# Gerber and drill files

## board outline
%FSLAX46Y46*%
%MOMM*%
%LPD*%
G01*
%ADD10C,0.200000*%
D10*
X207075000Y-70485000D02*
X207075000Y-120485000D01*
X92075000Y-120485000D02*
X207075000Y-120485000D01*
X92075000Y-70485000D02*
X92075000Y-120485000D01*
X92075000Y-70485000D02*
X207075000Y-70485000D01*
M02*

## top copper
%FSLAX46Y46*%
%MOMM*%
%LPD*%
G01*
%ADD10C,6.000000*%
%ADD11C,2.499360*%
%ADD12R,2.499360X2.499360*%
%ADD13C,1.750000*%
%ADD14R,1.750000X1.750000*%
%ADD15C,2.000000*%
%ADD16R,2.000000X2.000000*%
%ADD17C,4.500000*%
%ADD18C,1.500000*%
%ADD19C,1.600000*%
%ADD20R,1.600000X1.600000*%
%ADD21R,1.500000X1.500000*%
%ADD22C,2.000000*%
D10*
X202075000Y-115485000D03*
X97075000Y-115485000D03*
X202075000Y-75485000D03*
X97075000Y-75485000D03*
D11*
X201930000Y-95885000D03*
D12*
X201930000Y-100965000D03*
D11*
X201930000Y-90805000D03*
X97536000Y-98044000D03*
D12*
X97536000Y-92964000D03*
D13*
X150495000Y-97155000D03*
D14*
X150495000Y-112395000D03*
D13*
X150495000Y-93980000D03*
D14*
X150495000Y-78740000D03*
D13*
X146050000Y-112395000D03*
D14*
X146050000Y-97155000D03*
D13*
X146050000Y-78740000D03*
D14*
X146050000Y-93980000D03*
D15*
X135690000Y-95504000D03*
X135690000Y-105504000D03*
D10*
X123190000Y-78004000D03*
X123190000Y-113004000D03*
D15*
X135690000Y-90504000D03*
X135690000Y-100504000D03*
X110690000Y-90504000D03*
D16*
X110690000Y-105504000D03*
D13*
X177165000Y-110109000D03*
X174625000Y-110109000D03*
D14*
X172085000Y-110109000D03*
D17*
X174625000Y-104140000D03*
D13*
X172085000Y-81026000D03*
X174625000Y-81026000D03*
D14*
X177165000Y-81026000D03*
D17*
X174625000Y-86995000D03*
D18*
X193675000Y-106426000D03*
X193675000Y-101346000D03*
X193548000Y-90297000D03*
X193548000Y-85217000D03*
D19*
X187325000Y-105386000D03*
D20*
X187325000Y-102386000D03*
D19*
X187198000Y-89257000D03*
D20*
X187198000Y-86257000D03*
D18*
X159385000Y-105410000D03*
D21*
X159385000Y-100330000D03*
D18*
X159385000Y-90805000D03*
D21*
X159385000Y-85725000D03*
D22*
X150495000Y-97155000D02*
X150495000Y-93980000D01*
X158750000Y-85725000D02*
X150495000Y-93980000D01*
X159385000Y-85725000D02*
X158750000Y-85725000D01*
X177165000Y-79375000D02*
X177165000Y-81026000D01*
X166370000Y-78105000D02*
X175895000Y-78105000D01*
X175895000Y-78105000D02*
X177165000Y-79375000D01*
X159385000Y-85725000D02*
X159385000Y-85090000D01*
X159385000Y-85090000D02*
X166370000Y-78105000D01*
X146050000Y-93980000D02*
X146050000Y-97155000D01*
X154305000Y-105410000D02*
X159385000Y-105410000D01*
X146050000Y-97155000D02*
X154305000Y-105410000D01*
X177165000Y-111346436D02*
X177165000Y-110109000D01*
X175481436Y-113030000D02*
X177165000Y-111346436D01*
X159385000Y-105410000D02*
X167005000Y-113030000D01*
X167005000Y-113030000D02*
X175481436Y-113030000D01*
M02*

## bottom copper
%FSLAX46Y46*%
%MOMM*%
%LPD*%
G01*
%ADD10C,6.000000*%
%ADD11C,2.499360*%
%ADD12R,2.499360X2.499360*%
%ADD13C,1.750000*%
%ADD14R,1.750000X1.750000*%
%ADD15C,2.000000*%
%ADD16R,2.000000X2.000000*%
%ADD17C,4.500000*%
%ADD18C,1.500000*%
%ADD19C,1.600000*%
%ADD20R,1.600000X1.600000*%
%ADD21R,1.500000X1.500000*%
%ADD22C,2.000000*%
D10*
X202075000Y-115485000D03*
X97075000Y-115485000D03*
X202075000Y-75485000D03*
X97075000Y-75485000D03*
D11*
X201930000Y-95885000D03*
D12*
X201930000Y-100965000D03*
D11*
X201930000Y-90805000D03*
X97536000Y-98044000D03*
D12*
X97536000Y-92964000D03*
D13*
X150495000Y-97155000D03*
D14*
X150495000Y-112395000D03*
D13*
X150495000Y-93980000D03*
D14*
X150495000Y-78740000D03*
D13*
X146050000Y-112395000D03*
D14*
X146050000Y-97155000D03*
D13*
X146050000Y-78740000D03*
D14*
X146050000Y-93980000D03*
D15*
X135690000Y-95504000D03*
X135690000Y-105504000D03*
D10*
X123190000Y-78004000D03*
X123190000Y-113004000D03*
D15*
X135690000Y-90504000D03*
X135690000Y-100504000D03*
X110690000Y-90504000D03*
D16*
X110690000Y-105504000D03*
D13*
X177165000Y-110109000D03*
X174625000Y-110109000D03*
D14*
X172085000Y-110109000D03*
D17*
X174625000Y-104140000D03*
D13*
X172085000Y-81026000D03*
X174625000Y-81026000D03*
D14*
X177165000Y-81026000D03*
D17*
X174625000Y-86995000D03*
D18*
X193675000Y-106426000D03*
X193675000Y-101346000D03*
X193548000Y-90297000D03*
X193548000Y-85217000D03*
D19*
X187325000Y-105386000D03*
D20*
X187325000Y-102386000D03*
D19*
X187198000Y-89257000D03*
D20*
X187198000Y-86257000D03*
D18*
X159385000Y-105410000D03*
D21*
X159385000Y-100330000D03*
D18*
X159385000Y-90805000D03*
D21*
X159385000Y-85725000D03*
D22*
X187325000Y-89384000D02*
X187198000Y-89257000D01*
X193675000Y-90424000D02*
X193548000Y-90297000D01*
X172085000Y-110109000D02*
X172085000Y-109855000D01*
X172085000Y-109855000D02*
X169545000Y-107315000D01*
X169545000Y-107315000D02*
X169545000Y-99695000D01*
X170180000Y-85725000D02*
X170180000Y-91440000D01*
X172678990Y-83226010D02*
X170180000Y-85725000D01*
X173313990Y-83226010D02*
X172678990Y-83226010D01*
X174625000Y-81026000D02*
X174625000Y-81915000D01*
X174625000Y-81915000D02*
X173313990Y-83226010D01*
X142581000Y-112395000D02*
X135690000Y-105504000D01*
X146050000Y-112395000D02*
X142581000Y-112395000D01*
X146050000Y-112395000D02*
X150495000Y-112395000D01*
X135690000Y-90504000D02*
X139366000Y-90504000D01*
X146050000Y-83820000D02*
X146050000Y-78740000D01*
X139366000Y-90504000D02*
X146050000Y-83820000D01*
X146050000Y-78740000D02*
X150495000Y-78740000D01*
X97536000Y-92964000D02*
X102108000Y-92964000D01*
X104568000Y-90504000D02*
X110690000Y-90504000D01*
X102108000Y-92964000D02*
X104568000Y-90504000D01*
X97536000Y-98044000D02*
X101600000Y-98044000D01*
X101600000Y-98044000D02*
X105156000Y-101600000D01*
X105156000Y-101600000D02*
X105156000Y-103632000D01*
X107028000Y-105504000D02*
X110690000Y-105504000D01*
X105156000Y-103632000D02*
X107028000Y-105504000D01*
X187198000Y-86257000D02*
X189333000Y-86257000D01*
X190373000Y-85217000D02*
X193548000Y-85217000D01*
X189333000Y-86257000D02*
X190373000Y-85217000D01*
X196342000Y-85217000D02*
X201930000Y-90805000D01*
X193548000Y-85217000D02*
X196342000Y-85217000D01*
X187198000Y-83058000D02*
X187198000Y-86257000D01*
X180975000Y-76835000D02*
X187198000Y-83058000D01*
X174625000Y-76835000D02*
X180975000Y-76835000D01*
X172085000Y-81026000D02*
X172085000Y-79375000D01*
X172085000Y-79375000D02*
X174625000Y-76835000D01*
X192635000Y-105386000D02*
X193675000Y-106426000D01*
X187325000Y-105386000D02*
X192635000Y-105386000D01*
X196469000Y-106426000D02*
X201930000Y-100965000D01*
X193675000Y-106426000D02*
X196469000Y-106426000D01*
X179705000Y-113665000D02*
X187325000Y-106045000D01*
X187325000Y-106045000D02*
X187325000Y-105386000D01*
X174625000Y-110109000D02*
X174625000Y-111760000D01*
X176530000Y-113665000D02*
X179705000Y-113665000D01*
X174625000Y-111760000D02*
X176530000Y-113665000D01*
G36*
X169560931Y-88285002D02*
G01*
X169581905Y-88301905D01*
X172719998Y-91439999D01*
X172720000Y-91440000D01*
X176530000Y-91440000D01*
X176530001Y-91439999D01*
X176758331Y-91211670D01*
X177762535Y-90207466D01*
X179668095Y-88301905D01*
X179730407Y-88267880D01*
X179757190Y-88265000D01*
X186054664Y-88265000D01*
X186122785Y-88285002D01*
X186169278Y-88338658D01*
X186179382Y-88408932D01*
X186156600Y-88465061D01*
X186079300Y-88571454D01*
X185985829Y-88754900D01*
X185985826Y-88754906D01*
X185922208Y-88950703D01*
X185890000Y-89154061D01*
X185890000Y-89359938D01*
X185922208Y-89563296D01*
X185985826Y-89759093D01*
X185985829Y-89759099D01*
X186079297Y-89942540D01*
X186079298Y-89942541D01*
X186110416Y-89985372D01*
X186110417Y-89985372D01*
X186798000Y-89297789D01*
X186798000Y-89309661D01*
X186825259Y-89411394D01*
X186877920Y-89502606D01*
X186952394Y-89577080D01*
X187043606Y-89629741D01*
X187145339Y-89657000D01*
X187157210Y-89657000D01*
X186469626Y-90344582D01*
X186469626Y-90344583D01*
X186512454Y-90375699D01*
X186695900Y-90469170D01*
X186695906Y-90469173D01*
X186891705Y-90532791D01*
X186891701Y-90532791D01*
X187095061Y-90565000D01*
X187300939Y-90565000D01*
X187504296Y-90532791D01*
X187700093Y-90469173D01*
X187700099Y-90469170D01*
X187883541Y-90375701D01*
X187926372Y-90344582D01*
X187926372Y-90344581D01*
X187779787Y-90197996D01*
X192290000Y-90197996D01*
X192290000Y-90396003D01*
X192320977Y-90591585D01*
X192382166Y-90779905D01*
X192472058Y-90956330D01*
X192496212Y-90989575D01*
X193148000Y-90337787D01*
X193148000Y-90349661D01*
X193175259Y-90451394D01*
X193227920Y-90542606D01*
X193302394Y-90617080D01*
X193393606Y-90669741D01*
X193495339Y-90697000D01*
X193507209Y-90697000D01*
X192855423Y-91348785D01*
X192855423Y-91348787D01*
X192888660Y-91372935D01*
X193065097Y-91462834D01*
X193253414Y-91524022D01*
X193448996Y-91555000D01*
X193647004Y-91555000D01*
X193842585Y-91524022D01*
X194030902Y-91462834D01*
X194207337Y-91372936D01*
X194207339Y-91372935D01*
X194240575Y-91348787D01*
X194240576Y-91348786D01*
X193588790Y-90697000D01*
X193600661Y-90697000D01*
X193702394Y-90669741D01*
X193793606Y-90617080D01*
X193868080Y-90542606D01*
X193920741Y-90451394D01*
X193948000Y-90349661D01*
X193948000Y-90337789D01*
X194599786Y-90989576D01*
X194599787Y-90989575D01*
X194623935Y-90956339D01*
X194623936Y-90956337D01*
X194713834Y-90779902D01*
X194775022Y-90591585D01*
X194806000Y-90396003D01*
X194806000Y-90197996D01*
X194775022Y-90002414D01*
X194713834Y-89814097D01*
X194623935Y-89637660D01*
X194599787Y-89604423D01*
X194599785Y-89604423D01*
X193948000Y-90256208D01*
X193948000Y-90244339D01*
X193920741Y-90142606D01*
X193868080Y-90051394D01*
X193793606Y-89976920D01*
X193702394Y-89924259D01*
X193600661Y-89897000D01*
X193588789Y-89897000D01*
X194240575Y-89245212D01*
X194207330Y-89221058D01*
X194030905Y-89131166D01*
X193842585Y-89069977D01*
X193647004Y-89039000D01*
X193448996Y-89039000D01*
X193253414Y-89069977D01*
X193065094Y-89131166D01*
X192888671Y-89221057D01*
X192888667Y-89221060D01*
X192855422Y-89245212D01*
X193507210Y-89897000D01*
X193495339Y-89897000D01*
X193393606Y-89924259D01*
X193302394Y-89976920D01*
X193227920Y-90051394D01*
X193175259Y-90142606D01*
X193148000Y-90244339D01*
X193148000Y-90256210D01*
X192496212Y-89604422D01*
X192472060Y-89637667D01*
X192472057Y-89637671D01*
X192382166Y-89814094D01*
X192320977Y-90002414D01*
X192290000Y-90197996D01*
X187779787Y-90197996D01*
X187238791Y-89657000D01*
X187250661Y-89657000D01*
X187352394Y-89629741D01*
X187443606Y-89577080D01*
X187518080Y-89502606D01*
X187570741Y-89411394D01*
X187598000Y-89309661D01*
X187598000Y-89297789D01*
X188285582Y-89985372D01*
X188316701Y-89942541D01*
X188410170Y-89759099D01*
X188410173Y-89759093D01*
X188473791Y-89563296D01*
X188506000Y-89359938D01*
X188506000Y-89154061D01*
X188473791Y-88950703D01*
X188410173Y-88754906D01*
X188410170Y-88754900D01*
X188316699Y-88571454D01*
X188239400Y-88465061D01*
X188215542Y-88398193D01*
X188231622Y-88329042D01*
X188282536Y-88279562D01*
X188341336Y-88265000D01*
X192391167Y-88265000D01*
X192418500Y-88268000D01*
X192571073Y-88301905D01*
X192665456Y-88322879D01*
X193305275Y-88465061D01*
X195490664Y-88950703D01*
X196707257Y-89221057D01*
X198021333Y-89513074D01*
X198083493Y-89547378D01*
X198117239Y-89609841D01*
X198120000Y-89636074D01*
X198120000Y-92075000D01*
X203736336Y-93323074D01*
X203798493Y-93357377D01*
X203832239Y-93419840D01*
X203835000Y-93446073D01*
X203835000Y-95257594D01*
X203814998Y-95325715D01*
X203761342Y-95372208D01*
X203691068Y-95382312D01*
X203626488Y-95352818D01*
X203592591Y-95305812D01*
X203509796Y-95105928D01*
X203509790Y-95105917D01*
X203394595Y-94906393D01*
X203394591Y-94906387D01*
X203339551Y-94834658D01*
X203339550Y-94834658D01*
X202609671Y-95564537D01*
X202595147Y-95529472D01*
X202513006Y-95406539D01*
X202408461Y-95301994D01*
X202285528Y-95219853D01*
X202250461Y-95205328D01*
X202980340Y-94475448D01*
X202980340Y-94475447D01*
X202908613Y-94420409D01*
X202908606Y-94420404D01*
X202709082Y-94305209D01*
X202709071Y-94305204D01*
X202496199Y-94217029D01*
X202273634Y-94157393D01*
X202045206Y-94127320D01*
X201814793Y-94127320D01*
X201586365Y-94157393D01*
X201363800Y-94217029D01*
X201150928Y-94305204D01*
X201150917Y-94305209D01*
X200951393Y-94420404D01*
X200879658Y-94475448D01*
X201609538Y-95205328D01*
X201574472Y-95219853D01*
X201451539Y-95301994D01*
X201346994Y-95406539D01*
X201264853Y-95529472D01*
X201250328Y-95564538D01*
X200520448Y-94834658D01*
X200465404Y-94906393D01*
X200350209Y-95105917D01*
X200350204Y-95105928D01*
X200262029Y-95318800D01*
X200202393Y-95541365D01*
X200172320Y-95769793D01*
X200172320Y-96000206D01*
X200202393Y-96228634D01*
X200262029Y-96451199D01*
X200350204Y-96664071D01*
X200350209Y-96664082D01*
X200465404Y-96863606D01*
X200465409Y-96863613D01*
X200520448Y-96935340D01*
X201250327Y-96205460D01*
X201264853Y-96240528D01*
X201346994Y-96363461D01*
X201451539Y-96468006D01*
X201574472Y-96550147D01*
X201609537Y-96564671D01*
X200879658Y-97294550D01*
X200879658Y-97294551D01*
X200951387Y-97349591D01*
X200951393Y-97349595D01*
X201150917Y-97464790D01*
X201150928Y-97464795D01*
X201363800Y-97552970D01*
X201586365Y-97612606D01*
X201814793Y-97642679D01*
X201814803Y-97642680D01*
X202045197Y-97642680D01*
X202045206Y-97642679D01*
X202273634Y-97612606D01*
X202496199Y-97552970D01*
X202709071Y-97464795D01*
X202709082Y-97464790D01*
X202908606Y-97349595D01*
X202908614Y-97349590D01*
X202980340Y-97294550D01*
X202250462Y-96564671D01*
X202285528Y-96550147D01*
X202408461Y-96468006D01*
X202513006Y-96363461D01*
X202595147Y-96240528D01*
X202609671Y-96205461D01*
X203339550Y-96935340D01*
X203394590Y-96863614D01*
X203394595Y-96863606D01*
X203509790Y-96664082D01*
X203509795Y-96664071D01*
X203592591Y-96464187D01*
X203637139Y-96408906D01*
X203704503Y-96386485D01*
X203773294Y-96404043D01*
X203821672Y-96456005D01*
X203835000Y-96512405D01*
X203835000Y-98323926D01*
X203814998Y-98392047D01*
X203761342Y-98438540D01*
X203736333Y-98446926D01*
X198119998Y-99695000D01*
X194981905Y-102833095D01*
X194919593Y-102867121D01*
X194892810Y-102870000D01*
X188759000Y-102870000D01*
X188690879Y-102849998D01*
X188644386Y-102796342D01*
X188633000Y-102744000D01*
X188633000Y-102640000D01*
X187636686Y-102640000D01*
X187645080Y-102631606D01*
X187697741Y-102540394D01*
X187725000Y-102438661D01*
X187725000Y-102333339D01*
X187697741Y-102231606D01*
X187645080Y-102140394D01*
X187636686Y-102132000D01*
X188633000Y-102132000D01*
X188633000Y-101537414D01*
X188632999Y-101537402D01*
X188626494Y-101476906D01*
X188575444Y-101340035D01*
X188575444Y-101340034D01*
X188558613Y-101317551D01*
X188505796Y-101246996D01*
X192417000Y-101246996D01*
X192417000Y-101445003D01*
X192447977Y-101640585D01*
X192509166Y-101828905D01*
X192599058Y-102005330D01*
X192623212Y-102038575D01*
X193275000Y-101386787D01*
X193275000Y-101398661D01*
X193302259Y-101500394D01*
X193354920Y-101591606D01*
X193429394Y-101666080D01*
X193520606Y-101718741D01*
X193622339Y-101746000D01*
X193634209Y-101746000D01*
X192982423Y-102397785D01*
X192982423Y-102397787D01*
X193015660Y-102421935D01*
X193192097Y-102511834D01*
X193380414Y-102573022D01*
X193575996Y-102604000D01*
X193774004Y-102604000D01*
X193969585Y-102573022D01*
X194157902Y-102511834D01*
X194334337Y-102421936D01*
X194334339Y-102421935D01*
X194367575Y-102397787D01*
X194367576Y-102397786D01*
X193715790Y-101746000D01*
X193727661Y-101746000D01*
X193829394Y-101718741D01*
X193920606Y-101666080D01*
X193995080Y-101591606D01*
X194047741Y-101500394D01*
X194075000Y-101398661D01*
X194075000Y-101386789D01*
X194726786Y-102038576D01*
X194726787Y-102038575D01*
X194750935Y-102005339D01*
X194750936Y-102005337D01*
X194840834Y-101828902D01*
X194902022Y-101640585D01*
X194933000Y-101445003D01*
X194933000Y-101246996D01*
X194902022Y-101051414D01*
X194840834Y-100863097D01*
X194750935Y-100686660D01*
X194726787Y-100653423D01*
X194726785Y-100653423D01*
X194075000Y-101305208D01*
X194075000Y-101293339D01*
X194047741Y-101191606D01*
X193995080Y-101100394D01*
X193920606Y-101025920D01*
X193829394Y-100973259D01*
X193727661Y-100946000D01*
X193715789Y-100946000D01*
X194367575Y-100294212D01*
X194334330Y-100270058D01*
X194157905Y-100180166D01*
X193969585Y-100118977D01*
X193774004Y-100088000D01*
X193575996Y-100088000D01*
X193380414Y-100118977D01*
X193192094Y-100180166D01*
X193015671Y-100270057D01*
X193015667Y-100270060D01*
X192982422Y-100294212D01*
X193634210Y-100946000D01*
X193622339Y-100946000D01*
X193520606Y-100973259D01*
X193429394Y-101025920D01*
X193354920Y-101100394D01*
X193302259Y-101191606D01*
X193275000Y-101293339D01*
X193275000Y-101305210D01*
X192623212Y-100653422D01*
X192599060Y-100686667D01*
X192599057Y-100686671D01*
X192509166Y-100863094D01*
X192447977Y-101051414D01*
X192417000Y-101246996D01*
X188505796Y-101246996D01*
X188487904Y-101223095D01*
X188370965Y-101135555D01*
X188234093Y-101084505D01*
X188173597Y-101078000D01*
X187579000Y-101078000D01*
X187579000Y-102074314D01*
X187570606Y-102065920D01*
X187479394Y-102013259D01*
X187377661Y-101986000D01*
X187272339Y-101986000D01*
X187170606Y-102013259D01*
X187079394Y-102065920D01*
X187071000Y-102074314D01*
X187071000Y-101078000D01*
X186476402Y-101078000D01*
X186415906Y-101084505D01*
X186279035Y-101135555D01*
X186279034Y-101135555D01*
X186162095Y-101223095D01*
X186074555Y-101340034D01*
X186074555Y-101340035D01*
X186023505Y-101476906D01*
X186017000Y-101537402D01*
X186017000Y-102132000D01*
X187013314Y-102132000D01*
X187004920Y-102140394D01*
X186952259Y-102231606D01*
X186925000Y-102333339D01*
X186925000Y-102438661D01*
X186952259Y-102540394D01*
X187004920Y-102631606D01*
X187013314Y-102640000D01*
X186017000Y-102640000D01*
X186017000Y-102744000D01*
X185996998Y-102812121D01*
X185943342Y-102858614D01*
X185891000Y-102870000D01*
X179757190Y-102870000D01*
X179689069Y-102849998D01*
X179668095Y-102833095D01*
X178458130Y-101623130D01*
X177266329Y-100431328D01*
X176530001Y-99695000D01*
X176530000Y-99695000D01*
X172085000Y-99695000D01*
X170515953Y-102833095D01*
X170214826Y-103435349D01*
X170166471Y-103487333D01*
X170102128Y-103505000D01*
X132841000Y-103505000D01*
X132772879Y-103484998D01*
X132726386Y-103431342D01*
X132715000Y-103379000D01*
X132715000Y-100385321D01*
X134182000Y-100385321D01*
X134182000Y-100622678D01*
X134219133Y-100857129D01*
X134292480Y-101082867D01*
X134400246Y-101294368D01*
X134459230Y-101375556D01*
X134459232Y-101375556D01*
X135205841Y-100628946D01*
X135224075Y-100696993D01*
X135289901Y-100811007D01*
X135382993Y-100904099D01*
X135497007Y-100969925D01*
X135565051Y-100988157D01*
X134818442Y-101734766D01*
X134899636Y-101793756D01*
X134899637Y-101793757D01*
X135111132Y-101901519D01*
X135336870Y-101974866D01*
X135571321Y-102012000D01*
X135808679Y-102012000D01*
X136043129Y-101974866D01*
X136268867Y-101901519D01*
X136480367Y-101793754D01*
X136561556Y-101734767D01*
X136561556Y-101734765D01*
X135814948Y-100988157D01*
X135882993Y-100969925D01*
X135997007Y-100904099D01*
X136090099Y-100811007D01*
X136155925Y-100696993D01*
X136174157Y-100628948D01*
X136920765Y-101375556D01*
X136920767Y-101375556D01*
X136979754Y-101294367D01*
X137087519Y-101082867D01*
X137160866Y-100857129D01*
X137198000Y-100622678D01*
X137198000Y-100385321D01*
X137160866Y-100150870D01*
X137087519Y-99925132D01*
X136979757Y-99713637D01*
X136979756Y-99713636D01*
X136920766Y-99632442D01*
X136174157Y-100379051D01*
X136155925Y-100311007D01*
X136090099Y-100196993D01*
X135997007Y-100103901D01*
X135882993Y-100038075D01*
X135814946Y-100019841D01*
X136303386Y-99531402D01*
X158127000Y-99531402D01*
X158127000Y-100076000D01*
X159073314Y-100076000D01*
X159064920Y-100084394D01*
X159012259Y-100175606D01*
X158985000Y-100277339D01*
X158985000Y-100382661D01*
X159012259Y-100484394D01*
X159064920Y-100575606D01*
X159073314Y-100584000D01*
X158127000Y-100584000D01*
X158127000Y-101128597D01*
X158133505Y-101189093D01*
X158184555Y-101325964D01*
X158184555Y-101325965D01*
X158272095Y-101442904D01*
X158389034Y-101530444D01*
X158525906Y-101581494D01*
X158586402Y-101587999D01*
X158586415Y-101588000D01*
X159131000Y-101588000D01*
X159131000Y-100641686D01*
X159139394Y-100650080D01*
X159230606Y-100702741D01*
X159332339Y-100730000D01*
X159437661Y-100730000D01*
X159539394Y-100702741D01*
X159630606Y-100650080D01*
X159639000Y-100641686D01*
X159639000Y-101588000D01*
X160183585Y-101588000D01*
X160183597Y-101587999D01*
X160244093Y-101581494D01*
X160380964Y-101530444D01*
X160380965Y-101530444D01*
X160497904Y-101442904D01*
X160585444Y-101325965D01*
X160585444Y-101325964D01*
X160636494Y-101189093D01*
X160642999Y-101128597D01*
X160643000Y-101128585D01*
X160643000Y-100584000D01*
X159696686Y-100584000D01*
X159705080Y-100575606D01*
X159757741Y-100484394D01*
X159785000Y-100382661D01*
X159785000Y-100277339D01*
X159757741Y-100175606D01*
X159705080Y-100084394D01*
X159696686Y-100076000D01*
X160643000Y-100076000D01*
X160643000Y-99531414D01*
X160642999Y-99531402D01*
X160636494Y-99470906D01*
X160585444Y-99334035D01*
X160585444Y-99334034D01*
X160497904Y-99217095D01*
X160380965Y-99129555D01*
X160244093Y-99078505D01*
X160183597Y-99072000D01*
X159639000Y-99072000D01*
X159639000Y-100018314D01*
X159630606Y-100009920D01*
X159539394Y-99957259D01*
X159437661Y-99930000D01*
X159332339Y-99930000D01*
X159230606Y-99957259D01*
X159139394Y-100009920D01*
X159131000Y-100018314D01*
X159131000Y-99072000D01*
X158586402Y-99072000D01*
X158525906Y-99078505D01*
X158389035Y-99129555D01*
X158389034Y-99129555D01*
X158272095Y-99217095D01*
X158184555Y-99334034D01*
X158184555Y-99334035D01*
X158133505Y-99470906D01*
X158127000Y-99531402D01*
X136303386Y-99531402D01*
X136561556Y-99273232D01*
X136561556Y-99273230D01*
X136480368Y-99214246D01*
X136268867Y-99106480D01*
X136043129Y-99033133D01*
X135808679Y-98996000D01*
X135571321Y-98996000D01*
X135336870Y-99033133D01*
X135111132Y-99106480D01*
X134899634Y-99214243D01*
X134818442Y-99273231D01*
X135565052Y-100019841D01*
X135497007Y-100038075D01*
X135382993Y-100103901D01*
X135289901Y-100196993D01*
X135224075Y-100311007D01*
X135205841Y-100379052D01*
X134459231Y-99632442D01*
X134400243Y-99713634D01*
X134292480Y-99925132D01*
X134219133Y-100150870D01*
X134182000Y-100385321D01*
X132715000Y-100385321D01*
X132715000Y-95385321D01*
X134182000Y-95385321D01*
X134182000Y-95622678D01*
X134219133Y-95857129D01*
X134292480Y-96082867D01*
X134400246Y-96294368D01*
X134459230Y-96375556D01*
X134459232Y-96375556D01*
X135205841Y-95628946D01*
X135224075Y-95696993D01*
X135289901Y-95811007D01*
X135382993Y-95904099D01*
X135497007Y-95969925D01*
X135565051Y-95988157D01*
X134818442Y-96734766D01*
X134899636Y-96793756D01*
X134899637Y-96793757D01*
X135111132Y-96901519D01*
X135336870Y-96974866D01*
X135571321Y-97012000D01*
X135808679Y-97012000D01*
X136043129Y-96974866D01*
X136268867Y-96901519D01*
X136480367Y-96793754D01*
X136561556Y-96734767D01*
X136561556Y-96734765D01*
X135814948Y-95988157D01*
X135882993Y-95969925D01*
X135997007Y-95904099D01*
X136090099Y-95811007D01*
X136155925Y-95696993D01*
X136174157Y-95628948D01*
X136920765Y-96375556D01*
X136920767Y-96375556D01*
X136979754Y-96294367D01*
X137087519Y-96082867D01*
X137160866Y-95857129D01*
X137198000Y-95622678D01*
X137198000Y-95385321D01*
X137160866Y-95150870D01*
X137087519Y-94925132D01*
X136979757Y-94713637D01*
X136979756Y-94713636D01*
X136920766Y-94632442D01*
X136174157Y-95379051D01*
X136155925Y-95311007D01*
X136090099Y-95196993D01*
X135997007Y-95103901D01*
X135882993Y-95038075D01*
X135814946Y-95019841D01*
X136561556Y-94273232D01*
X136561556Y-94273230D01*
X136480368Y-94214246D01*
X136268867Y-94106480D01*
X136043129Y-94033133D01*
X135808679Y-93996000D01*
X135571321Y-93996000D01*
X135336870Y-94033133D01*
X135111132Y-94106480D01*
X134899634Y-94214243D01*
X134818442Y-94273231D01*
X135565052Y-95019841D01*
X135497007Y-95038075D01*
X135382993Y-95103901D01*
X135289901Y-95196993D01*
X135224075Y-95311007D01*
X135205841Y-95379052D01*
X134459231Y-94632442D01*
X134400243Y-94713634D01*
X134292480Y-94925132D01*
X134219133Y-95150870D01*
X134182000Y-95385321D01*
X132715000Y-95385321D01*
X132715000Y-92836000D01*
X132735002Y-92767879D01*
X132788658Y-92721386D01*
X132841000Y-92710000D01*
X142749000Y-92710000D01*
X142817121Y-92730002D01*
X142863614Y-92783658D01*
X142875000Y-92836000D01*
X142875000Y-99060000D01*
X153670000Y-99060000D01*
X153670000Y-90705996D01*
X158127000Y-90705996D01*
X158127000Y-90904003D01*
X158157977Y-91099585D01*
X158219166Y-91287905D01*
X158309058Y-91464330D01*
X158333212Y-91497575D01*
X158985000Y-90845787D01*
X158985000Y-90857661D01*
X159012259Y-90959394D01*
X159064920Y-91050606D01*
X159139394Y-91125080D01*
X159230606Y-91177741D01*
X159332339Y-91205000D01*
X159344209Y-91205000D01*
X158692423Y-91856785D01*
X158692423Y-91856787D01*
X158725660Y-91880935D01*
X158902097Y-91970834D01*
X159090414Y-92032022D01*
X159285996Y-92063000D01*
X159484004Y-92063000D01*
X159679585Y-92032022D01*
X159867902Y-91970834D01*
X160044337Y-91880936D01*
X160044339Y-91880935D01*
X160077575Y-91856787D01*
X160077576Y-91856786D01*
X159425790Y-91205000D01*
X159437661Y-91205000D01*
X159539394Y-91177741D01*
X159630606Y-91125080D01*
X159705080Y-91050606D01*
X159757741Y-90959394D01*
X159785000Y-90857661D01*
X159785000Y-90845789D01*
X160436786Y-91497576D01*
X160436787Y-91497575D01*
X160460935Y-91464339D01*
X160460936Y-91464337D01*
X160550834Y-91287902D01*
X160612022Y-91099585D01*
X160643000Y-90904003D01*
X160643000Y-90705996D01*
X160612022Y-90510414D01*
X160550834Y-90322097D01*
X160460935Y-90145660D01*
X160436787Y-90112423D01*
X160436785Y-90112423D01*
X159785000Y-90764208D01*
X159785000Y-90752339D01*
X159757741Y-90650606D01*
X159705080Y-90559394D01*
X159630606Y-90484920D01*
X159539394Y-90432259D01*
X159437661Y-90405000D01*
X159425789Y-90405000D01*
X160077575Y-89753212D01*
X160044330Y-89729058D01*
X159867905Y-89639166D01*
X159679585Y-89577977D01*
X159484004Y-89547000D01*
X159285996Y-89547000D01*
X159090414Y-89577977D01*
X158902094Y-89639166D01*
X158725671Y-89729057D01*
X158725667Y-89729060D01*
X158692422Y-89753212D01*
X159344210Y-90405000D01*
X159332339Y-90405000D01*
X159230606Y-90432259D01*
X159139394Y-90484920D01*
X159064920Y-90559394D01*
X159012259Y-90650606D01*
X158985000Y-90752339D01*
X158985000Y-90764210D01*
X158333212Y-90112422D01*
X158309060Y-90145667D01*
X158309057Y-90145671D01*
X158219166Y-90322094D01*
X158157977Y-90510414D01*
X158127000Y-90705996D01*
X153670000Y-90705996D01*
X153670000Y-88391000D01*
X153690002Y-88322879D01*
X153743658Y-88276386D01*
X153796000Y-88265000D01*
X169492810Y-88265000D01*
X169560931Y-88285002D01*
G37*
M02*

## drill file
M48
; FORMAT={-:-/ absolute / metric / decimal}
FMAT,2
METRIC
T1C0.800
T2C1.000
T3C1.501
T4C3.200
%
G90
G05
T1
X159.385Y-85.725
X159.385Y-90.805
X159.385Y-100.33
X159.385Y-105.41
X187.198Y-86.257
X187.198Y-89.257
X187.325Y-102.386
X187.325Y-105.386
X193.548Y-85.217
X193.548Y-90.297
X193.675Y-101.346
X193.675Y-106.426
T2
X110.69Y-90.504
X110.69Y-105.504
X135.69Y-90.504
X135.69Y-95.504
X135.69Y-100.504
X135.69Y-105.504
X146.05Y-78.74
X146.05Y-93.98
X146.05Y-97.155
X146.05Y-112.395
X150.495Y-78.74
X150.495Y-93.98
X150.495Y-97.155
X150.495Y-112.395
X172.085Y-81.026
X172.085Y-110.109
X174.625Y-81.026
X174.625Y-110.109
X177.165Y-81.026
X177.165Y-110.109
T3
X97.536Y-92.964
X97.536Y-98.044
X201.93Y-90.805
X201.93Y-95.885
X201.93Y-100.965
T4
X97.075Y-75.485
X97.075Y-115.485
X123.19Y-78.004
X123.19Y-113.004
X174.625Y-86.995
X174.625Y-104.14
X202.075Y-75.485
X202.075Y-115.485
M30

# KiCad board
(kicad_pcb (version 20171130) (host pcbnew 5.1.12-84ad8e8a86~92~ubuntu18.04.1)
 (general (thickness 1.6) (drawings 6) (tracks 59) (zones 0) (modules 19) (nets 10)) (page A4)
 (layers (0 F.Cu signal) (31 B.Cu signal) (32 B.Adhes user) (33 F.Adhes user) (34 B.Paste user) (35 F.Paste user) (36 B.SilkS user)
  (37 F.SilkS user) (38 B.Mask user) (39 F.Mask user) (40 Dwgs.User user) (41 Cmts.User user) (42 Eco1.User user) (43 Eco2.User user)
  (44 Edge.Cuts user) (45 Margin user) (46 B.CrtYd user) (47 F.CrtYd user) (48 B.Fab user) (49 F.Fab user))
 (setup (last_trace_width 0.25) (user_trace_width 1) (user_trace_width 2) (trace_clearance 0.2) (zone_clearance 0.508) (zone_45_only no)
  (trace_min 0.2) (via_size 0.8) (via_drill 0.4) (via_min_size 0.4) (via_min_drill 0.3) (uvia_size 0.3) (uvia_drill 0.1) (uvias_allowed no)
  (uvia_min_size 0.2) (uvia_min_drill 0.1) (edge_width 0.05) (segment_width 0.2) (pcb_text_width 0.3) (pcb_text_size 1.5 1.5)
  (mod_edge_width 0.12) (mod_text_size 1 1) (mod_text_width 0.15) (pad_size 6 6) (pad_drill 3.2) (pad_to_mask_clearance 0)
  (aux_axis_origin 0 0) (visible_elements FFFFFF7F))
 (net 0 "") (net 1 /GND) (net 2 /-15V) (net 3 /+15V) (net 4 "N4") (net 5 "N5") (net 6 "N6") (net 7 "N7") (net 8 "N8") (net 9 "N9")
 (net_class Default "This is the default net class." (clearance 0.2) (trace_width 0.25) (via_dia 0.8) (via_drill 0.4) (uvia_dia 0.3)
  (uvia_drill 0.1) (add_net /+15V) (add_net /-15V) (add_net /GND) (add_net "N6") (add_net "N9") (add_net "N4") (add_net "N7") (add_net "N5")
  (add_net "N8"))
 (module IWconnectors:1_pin (layer F.Cu) (at 202.075 115.485)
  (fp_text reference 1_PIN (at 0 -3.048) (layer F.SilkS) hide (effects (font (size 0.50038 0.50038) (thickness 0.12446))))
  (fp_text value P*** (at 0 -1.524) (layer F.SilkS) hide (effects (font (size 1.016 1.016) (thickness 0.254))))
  (pad 1 thru_hole circle (at 0 0) (size 6 6) (drill 3.2) (layers *.Cu *.Mask)))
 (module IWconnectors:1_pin (layer F.Cu) (at 97.075 115.485)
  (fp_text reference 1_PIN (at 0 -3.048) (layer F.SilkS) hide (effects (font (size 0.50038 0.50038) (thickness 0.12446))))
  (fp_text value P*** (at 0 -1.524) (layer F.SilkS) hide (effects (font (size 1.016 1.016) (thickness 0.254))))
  (pad 1 thru_hole circle (at 0 0) (size 6 6) (drill 3.2) (layers *.Cu *.Mask)))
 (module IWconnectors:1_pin (layer F.Cu) (at 202.075 75.485)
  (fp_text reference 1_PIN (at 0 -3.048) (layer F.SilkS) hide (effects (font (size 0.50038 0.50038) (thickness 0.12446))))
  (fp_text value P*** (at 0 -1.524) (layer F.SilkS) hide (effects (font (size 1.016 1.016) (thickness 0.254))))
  (pad 1 thru_hole circle (at 0 0) (size 6 6) (drill 3.2) (layers *.Cu *.Mask)))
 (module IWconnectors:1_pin (layer F.Cu) (at 97.075 75.485)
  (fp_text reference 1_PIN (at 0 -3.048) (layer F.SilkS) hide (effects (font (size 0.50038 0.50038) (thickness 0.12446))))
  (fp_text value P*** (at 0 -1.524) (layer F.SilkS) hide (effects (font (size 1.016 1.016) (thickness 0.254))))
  (pad 1 thru_hole circle (at 0 0) (size 6 6) (drill 3.2) (layers *.Cu *.Mask)))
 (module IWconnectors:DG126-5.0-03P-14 (layer F.Cu) (at 201.93 95.885 90)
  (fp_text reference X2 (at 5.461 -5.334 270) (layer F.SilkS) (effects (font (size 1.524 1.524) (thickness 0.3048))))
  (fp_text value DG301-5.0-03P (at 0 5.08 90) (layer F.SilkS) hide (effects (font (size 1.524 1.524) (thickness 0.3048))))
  (pad 2 thru_hole circle (at 0 0 90) (size 2.49936 2.49936) (drill 1.50114) (layers *.Cu *.Mask) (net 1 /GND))
  (pad 1 thru_hole rect (at -5.08 0 90) (size 2.49936 2.49936) (drill 1.50114) (layers *.Cu *.Mask) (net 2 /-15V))
  (pad 3 thru_hole circle (at 5.08 0 90) (size 2.49936 2.49936) (drill 1.50114) (layers *.Cu *.Mask) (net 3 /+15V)))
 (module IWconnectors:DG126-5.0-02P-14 (layer F.Cu) (at 97.536 95.504 270)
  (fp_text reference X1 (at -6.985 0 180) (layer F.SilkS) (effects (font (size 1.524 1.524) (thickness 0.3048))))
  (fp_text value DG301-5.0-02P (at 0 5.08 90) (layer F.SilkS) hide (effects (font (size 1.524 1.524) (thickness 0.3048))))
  (pad 2 thru_hole circle (at 2.54 0 270) (size 2.49936 2.49936) (drill 1.50114) (layers *.Cu *.Mask) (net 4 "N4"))
  (pad 1 thru_hole rect (at -2.54 0 270) (size 2.49936 2.49936) (drill 1.50114) (layers *.Cu *.Mask) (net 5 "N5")))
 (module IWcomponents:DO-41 (layer F.Cu) (at 150.495 97.155 270)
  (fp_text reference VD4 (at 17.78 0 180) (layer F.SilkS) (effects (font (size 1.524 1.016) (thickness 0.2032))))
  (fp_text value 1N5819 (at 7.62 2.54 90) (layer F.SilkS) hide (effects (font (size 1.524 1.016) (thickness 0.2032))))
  (pad 2 thru_hole circle (at 0 0 270) (size 1.75 1.75) (drill 1) (layers *.Cu *.Mask) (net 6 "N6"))
  (pad 1 thru_hole rect (at 15.24 0 270) (size 1.75 1.75) (drill 1) (layers *.Cu *.Mask) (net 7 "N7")))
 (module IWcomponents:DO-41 (layer F.Cu) (at 150.495 93.98 90)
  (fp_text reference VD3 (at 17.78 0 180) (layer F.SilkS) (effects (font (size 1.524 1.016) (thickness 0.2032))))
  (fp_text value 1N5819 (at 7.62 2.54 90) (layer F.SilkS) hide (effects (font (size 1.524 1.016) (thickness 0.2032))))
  (pad 2 thru_hole circle (at 0 0 90) (size 1.75 1.75) (drill 1) (layers *.Cu *.Mask) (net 6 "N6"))
  (pad 1 thru_hole rect (at 15.24 0 90) (size 1.75 1.75) (drill 1) (layers *.Cu *.Mask) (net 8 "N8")))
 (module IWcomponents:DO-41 (layer F.Cu) (at 146.05 112.395 90)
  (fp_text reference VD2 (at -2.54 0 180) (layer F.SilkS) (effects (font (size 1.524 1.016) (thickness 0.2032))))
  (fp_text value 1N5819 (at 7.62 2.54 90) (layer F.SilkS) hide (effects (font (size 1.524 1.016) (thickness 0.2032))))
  (pad 2 thru_hole circle (at 0 0 90) (size 1.75 1.75) (drill 1) (layers *.Cu *.Mask) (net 7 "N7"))
  (pad 1 thru_hole rect (at 15.24 0 90) (size 1.75 1.75) (drill 1) (layers *.Cu *.Mask) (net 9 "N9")))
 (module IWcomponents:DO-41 (layer F.Cu) (at 146.05 78.74 270)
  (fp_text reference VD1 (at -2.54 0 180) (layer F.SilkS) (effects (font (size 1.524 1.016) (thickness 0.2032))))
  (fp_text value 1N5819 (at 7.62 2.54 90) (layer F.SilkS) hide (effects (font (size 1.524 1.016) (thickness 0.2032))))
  (pad 2 thru_hole circle (at 0 0 270) (size 1.75 1.75) (drill 1) (layers *.Cu *.Mask) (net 8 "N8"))
  (pad 1 thru_hole rect (at 15.24 0 270) (size 1.75 1.75) (drill 1) (layers *.Cu *.Mask) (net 9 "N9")))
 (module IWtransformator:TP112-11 (layer F.Cu) (at 123.19 95.504 90)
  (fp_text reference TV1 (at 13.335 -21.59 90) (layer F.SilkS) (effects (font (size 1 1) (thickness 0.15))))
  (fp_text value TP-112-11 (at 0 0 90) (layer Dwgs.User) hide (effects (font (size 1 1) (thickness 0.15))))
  (pad 8 thru_hole circle (at 0 12.5 90) (size 2 2) (drill 1) (layers *.Cu *.Mask) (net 1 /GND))
  (pad 10 thru_hole circle (at -10 12.5 90) (size 2 2) (drill 1) (layers *.Cu *.Mask) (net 7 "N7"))
  (pad ~ thru_hole circle (at 17.5 0 90) (size 6 6) (drill 3.2) (layers *.Cu *.Mask))
  (pad ~ thru_hole circle (at -17.5 0 90) (size 6 6) (drill 3.2) (layers *.Cu *.Mask))
  (pad 7 thru_hole circle (at 5 12.5 90) (size 2 2) (drill 1) (layers *.Cu *.Mask) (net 8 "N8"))
  (pad 9 thru_hole circle (at -5 12.5 90) (size 2 2) (drill 1) (layers *.Cu *.Mask) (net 1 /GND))
  (pad 4 thru_hole circle (at 5 -12.5 90) (size 2 2) (drill 1) (layers *.Cu *.Mask) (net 5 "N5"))
  (pad 1 thru_hole rect (at -10 -12.5 90) (size 2 2) (drill 1) (layers *.Cu *.Mask) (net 4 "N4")))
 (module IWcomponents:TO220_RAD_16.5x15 (layer F.Cu) (at 174.625 104.14 90)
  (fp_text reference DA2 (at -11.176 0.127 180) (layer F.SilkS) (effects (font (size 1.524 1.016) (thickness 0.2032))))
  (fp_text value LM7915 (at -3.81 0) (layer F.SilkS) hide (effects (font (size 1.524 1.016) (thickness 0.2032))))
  (pad 3 thru_hole circle (at -5.969 2.54 90) (size 1.75 1.75) (drill 1) (layers *.Cu *.Mask) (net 9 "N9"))
  (pad 2 thru_hole circle (at -5.969 0 90) (size 1.75 1.75) (drill 1) (layers *.Cu *.Mask) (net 2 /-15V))
  (pad 1 thru_hole rect (at -5.969 -2.54 90) (size 1.75 1.75) (drill 1) (layers *.Cu *.Mask) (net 1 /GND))
  (pad 4 thru_hole circle (at 0 0 90) (size 4.5 4.5) (drill 3.2) (layers *.Cu *.Mask)))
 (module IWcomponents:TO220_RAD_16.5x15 (layer F.Cu) (at 174.625 86.995 270)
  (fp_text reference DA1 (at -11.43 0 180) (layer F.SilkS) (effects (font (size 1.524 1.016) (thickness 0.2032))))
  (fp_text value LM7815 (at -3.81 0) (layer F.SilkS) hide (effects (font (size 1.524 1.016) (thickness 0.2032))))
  (pad 3 thru_hole circle (at -5.969 2.54 270) (size 1.75 1.75) (drill 1) (layers *.Cu *.Mask) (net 3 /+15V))
  (pad 2 thru_hole circle (at -5.969 0 270) (size 1.75 1.75) (drill 1) (layers *.Cu *.Mask) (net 1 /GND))
  (pad 1 thru_hole rect (at -5.969 -2.54 270) (size 1.75 1.75) (drill 1) (layers *.Cu *.Mask) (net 6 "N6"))
  (pad 4 thru_hole circle (at 0 0 270) (size 4.5 4.5) (drill 3.2) (layers *.Cu *.Mask)))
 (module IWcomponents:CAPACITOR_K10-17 (layer F.Cu) (at 193.675 103.886 270)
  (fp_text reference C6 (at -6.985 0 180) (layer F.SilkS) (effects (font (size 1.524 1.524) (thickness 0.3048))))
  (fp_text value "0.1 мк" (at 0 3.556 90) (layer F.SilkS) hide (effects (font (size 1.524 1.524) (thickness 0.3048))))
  (pad 2 thru_hole circle (at 2.54 0 270) (size 1.5 1.5) (drill 0.8) (layers *.Cu *.Mask) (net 2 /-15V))
  (pad 1 thru_hole circle (at -2.54 0 270) (size 1.5 1.5) (drill 0.8) (layers *.Cu *.Mask) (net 1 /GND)))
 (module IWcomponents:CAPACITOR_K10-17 (layer F.Cu) (at 193.548 87.757 270)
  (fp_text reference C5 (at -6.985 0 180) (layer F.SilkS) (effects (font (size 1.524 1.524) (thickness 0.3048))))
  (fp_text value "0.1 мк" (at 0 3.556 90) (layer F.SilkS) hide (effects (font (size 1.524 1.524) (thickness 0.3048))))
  (pad 2 thru_hole circle (at 2.54 0 270) (size 1.5 1.5) (drill 0.8) (layers *.Cu *.Mask) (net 1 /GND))
  (pad 1 thru_hole circle (at -2.54 0 270) (size 1.5 1.5) (drill 0.8) (layers *.Cu *.Mask) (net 3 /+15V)))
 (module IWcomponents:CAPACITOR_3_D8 (layer F.Cu) (at 187.325 103.886 270)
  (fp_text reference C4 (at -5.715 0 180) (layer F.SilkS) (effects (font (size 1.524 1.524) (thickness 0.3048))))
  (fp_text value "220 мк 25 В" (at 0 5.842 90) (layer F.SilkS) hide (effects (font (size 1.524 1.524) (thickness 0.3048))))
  (pad 2 thru_hole circle (at 1.5 0 270) (size 1.6 1.6) (drill 0.8) (layers *.Cu *.Mask) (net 2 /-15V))
  (pad 1 thru_hole rect (at -1.5 0 270) (size 1.6 1.6) (drill 0.8) (layers *.Cu *.Mask) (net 1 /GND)))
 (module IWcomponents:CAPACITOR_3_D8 (layer F.Cu) (at 187.198 87.757 270)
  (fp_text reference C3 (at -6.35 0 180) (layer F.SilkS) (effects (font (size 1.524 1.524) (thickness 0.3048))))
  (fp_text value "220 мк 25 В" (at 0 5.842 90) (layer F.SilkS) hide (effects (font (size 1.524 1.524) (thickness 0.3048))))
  (pad 2 thru_hole circle (at 1.5 0 270) (size 1.6 1.6) (drill 0.8) (layers *.Cu *.Mask) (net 1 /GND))
  (pad 1 thru_hole rect (at -1.5 0 270) (size 1.6 1.6) (drill 0.8) (layers *.Cu *.Mask) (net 3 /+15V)))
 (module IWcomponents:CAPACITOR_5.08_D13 (layer F.Cu) (at 159.385 102.87 270)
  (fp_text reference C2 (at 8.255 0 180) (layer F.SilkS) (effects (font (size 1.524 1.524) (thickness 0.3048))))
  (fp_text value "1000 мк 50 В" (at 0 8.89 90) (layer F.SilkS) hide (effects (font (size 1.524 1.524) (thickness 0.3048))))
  (pad 2 thru_hole circle (at 2.54 0 270) (size 1.5 1.5) (drill 0.8) (layers *.Cu *.Mask) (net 9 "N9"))
  (pad 1 thru_hole rect (at -2.54 0 270) (size 1.5 1.5) (drill 0.8) (layers *.Cu *.Mask) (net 1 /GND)))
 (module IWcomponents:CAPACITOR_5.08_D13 (layer F.Cu) (at 159.385 88.265 270)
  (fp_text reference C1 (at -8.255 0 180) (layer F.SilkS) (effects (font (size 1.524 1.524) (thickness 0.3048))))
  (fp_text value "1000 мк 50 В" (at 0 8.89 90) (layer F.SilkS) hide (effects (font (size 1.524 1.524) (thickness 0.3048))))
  (pad 2 thru_hole circle (at 2.54 0 270) (size 1.5 1.5) (drill 0.8) (layers *.Cu *.Mask) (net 1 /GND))
  (pad 1 thru_hole rect (at -2.54 0 270) (size 1.5 1.5) (drill 0.8) (layers *.Cu *.Mask) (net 6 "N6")))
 (gr_line (start 207.075 70.485) (end 207.075 120.485) (layer Edge.Cuts) (width 0.2))
 (gr_line (start 92.075 120.485) (end 207.075 120.485) (layer Edge.Cuts) (width 0.2))
 (gr_line (start 92.075 70.485) (end 92.075 120.485) (layer Edge.Cuts) (width 0.2))
 (gr_line (start 92.075 70.485) (end 207.075 70.485) (layer Edge.Cuts) (width 0.2))
 (segment (start 187.325 89.384) (end 187.198 89.257) (width 2) (layer B.Cu) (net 1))
 (segment (start 193.675 90.424) (end 193.548 90.297) (width 2) (layer B.Cu) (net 1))
 (segment (start 172.085 110.109) (end 172.085 109.855) (width 2) (layer B.Cu) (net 1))
 (segment (start 172.085 109.855) (end 169.545 107.315) (width 2) (layer B.Cu) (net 1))
 (segment (start 169.545 107.315) (end 169.545 99.695) (width 2) (layer B.Cu) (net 1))
 (segment (start 170.18 85.725) (end 170.18 91.44) (width 2) (layer B.Cu) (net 1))
 (segment (start 172.67899 83.22601) (end 170.18 85.725) (width 2) (layer B.Cu) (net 1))
 (segment (start 173.31399 83.22601) (end 172.67899 83.22601) (width 2) (layer B.Cu) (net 1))
 (segment (start 174.625 81.026) (end 174.625 81.915) (width 2) (layer B.Cu) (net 1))
 (segment (start 174.625 81.915) (end 173.31399 83.22601) (width 2) (layer B.Cu) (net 1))
 (segment (start 150.495 97.155) (end 150.495 93.98) (width 2) (layer F.Cu) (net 6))
 (segment (start 158.75 85.725) (end 150.495 93.98) (width 2) (layer F.Cu) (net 6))
 (segment (start 159.385 85.725) (end 158.75 85.725) (width 2) (layer F.Cu) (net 6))
 (segment (start 177.165 79.375) (end 177.165 81.026) (width 2) (layer F.Cu) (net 6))
 (segment (start 166.37 78.105) (end 175.895 78.105) (width 2) (layer F.Cu) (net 6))
 (segment (start 175.895 78.105) (end 177.165 79.375) (width 2) (layer F.Cu) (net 6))
 (segment (start 159.385 85.725) (end 159.385 85.09) (width 2) (layer F.Cu) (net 6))
 (segment (start 159.385 85.09) (end 166.37 78.105) (width 2) (layer F.Cu) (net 6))
 (segment (start 146.05 93.98) (end 146.05 97.155) (width 2) (layer F.Cu) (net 9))
 (segment (start 154.305 105.41) (end 159.385 105.41) (width 2) (layer F.Cu) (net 9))
 (segment (start 146.05 97.155) (end 154.305 105.41) (width 2) (layer F.Cu) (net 9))
 (segment (start 177.165 111.346436) (end 177.165 110.109) (width 2) (layer F.Cu) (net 9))
 (segment (start 175.481436 113.03) (end 177.165 111.346436) (width 2) (layer F.Cu) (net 9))
 (segment (start 159.385 105.41) (end 167.005 113.03) (width 2) (layer F.Cu) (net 9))
 (segment (start 167.005 113.03) (end 175.481436 113.03) (width 2) (layer F.Cu) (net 9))
 (segment (start 142.581 112.395) (end 135.69 105.504) (width 2) (layer B.Cu) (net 7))
 (segment (start 146.05 112.395) (end 142.581 112.395) (width 2) (layer B.Cu) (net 7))
 (segment (start 146.05 112.395) (end 150.495 112.395) (width 2) (layer B.Cu) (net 7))
 (segment (start 135.69 90.504) (end 139.366 90.504) (width 2) (layer B.Cu) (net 8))
 (segment (start 146.05 83.82) (end 146.05 78.74) (width 2) (layer B.Cu) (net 8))
 (segment (start 139.366 90.504) (end 146.05 83.82) (width 2) (layer B.Cu) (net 8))
 (segment (start 146.05 78.74) (end 150.495 78.74) (width 2) (layer B.Cu) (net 8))
 (segment (start 97.536 92.964) (end 102.108 92.964) (width 2) (layer B.Cu) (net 5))
 (segment (start 104.568 90.504) (end 110.69 90.504) (width 2) (layer B.Cu) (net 5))
 (segment (start 102.108 92.964) (end 104.568 90.504) (width 2) (layer B.Cu) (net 5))
 (segment (start 97.536 98.044) (end 101.6 98.044) (width 2) (layer B.Cu) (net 4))
 (segment (start 101.6 98.044) (end 105.156 101.6) (width 2) (layer B.Cu) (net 4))
 (segment (start 105.156 101.6) (end 105.156 103.632) (width 2) (layer B.Cu) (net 4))
 (segment (start 107.028 105.504) (end 110.69 105.504) (width 2) (layer B.Cu) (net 4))
 (segment (start 105.156 103.632) (end 107.028 105.504) (width 2) (layer B.Cu) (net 4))
 (segment (start 187.198 86.257) (end 189.333 86.257) (width 2) (layer B.Cu) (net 3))
 (segment (start 190.373 85.217) (end 193.548 85.217) (width 2) (layer B.Cu) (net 3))
 (segment (start 189.333 86.257) (end 190.373 85.217) (width 2) (layer B.Cu) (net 3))
 (segment (start 196.342 85.217) (end 201.93 90.805) (width 2) (layer B.Cu) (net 3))
 (segment (start 193.548 85.217) (end 196.342 85.217) (width 2) (layer B.Cu) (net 3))
 (segment (start 187.198 83.058) (end 187.198 86.257) (width 2) (layer B.Cu) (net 3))
 (segment (start 180.975 76.835) (end 187.198 83.058) (width 2) (layer B.Cu) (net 3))
 (segment (start 174.625 76.835) (end 180.975 76.835) (width 2) (layer B.Cu) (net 3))
 (segment (start 172.085 81.026) (end 172.085 79.375) (width 2) (layer B.Cu) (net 3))
 (segment (start 172.085 79.375) (end 174.625 76.835) (width 2) (layer B.Cu) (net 3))
 (segment (start 192.635 105.386) (end 193.675 106.426) (width 2) (layer B.Cu) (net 2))
 (segment (start 187.325 105.386) (end 192.635 105.386) (width 2) (layer B.Cu) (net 2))
 (segment (start 196.469 106.426) (end 201.93 100.965) (width 2) (layer B.Cu) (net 2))
 (segment (start 193.675 106.426) (end 196.469 106.426) (width 2) (layer B.Cu) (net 2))
 (segment (start 179.705 113.665) (end 187.325 106.045) (width 2) (layer B.Cu) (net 2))
 (segment (start 187.325 106.045) (end 187.325 105.386) (width 2) (layer B.Cu) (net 2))
 (segment (start 174.625 110.109) (end 174.625 111.76) (width 2) (layer B.Cu) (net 2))
 (segment (start 176.53 113.665) (end 179.705 113.665) (width 2) (layer B.Cu) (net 2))
 (segment (start 174.625 111.76) (end 176.53 113.665) (width 2) (layer B.Cu) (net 2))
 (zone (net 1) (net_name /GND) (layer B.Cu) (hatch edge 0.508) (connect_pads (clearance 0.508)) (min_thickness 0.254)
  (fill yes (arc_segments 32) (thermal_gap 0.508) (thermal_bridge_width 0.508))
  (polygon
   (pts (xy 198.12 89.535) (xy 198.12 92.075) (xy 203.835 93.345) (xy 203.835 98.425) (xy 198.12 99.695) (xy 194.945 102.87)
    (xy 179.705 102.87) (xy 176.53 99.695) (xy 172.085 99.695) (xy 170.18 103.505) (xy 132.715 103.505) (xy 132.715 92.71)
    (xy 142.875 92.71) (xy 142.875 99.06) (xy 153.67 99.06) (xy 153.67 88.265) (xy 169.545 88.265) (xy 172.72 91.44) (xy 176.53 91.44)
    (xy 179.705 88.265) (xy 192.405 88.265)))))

